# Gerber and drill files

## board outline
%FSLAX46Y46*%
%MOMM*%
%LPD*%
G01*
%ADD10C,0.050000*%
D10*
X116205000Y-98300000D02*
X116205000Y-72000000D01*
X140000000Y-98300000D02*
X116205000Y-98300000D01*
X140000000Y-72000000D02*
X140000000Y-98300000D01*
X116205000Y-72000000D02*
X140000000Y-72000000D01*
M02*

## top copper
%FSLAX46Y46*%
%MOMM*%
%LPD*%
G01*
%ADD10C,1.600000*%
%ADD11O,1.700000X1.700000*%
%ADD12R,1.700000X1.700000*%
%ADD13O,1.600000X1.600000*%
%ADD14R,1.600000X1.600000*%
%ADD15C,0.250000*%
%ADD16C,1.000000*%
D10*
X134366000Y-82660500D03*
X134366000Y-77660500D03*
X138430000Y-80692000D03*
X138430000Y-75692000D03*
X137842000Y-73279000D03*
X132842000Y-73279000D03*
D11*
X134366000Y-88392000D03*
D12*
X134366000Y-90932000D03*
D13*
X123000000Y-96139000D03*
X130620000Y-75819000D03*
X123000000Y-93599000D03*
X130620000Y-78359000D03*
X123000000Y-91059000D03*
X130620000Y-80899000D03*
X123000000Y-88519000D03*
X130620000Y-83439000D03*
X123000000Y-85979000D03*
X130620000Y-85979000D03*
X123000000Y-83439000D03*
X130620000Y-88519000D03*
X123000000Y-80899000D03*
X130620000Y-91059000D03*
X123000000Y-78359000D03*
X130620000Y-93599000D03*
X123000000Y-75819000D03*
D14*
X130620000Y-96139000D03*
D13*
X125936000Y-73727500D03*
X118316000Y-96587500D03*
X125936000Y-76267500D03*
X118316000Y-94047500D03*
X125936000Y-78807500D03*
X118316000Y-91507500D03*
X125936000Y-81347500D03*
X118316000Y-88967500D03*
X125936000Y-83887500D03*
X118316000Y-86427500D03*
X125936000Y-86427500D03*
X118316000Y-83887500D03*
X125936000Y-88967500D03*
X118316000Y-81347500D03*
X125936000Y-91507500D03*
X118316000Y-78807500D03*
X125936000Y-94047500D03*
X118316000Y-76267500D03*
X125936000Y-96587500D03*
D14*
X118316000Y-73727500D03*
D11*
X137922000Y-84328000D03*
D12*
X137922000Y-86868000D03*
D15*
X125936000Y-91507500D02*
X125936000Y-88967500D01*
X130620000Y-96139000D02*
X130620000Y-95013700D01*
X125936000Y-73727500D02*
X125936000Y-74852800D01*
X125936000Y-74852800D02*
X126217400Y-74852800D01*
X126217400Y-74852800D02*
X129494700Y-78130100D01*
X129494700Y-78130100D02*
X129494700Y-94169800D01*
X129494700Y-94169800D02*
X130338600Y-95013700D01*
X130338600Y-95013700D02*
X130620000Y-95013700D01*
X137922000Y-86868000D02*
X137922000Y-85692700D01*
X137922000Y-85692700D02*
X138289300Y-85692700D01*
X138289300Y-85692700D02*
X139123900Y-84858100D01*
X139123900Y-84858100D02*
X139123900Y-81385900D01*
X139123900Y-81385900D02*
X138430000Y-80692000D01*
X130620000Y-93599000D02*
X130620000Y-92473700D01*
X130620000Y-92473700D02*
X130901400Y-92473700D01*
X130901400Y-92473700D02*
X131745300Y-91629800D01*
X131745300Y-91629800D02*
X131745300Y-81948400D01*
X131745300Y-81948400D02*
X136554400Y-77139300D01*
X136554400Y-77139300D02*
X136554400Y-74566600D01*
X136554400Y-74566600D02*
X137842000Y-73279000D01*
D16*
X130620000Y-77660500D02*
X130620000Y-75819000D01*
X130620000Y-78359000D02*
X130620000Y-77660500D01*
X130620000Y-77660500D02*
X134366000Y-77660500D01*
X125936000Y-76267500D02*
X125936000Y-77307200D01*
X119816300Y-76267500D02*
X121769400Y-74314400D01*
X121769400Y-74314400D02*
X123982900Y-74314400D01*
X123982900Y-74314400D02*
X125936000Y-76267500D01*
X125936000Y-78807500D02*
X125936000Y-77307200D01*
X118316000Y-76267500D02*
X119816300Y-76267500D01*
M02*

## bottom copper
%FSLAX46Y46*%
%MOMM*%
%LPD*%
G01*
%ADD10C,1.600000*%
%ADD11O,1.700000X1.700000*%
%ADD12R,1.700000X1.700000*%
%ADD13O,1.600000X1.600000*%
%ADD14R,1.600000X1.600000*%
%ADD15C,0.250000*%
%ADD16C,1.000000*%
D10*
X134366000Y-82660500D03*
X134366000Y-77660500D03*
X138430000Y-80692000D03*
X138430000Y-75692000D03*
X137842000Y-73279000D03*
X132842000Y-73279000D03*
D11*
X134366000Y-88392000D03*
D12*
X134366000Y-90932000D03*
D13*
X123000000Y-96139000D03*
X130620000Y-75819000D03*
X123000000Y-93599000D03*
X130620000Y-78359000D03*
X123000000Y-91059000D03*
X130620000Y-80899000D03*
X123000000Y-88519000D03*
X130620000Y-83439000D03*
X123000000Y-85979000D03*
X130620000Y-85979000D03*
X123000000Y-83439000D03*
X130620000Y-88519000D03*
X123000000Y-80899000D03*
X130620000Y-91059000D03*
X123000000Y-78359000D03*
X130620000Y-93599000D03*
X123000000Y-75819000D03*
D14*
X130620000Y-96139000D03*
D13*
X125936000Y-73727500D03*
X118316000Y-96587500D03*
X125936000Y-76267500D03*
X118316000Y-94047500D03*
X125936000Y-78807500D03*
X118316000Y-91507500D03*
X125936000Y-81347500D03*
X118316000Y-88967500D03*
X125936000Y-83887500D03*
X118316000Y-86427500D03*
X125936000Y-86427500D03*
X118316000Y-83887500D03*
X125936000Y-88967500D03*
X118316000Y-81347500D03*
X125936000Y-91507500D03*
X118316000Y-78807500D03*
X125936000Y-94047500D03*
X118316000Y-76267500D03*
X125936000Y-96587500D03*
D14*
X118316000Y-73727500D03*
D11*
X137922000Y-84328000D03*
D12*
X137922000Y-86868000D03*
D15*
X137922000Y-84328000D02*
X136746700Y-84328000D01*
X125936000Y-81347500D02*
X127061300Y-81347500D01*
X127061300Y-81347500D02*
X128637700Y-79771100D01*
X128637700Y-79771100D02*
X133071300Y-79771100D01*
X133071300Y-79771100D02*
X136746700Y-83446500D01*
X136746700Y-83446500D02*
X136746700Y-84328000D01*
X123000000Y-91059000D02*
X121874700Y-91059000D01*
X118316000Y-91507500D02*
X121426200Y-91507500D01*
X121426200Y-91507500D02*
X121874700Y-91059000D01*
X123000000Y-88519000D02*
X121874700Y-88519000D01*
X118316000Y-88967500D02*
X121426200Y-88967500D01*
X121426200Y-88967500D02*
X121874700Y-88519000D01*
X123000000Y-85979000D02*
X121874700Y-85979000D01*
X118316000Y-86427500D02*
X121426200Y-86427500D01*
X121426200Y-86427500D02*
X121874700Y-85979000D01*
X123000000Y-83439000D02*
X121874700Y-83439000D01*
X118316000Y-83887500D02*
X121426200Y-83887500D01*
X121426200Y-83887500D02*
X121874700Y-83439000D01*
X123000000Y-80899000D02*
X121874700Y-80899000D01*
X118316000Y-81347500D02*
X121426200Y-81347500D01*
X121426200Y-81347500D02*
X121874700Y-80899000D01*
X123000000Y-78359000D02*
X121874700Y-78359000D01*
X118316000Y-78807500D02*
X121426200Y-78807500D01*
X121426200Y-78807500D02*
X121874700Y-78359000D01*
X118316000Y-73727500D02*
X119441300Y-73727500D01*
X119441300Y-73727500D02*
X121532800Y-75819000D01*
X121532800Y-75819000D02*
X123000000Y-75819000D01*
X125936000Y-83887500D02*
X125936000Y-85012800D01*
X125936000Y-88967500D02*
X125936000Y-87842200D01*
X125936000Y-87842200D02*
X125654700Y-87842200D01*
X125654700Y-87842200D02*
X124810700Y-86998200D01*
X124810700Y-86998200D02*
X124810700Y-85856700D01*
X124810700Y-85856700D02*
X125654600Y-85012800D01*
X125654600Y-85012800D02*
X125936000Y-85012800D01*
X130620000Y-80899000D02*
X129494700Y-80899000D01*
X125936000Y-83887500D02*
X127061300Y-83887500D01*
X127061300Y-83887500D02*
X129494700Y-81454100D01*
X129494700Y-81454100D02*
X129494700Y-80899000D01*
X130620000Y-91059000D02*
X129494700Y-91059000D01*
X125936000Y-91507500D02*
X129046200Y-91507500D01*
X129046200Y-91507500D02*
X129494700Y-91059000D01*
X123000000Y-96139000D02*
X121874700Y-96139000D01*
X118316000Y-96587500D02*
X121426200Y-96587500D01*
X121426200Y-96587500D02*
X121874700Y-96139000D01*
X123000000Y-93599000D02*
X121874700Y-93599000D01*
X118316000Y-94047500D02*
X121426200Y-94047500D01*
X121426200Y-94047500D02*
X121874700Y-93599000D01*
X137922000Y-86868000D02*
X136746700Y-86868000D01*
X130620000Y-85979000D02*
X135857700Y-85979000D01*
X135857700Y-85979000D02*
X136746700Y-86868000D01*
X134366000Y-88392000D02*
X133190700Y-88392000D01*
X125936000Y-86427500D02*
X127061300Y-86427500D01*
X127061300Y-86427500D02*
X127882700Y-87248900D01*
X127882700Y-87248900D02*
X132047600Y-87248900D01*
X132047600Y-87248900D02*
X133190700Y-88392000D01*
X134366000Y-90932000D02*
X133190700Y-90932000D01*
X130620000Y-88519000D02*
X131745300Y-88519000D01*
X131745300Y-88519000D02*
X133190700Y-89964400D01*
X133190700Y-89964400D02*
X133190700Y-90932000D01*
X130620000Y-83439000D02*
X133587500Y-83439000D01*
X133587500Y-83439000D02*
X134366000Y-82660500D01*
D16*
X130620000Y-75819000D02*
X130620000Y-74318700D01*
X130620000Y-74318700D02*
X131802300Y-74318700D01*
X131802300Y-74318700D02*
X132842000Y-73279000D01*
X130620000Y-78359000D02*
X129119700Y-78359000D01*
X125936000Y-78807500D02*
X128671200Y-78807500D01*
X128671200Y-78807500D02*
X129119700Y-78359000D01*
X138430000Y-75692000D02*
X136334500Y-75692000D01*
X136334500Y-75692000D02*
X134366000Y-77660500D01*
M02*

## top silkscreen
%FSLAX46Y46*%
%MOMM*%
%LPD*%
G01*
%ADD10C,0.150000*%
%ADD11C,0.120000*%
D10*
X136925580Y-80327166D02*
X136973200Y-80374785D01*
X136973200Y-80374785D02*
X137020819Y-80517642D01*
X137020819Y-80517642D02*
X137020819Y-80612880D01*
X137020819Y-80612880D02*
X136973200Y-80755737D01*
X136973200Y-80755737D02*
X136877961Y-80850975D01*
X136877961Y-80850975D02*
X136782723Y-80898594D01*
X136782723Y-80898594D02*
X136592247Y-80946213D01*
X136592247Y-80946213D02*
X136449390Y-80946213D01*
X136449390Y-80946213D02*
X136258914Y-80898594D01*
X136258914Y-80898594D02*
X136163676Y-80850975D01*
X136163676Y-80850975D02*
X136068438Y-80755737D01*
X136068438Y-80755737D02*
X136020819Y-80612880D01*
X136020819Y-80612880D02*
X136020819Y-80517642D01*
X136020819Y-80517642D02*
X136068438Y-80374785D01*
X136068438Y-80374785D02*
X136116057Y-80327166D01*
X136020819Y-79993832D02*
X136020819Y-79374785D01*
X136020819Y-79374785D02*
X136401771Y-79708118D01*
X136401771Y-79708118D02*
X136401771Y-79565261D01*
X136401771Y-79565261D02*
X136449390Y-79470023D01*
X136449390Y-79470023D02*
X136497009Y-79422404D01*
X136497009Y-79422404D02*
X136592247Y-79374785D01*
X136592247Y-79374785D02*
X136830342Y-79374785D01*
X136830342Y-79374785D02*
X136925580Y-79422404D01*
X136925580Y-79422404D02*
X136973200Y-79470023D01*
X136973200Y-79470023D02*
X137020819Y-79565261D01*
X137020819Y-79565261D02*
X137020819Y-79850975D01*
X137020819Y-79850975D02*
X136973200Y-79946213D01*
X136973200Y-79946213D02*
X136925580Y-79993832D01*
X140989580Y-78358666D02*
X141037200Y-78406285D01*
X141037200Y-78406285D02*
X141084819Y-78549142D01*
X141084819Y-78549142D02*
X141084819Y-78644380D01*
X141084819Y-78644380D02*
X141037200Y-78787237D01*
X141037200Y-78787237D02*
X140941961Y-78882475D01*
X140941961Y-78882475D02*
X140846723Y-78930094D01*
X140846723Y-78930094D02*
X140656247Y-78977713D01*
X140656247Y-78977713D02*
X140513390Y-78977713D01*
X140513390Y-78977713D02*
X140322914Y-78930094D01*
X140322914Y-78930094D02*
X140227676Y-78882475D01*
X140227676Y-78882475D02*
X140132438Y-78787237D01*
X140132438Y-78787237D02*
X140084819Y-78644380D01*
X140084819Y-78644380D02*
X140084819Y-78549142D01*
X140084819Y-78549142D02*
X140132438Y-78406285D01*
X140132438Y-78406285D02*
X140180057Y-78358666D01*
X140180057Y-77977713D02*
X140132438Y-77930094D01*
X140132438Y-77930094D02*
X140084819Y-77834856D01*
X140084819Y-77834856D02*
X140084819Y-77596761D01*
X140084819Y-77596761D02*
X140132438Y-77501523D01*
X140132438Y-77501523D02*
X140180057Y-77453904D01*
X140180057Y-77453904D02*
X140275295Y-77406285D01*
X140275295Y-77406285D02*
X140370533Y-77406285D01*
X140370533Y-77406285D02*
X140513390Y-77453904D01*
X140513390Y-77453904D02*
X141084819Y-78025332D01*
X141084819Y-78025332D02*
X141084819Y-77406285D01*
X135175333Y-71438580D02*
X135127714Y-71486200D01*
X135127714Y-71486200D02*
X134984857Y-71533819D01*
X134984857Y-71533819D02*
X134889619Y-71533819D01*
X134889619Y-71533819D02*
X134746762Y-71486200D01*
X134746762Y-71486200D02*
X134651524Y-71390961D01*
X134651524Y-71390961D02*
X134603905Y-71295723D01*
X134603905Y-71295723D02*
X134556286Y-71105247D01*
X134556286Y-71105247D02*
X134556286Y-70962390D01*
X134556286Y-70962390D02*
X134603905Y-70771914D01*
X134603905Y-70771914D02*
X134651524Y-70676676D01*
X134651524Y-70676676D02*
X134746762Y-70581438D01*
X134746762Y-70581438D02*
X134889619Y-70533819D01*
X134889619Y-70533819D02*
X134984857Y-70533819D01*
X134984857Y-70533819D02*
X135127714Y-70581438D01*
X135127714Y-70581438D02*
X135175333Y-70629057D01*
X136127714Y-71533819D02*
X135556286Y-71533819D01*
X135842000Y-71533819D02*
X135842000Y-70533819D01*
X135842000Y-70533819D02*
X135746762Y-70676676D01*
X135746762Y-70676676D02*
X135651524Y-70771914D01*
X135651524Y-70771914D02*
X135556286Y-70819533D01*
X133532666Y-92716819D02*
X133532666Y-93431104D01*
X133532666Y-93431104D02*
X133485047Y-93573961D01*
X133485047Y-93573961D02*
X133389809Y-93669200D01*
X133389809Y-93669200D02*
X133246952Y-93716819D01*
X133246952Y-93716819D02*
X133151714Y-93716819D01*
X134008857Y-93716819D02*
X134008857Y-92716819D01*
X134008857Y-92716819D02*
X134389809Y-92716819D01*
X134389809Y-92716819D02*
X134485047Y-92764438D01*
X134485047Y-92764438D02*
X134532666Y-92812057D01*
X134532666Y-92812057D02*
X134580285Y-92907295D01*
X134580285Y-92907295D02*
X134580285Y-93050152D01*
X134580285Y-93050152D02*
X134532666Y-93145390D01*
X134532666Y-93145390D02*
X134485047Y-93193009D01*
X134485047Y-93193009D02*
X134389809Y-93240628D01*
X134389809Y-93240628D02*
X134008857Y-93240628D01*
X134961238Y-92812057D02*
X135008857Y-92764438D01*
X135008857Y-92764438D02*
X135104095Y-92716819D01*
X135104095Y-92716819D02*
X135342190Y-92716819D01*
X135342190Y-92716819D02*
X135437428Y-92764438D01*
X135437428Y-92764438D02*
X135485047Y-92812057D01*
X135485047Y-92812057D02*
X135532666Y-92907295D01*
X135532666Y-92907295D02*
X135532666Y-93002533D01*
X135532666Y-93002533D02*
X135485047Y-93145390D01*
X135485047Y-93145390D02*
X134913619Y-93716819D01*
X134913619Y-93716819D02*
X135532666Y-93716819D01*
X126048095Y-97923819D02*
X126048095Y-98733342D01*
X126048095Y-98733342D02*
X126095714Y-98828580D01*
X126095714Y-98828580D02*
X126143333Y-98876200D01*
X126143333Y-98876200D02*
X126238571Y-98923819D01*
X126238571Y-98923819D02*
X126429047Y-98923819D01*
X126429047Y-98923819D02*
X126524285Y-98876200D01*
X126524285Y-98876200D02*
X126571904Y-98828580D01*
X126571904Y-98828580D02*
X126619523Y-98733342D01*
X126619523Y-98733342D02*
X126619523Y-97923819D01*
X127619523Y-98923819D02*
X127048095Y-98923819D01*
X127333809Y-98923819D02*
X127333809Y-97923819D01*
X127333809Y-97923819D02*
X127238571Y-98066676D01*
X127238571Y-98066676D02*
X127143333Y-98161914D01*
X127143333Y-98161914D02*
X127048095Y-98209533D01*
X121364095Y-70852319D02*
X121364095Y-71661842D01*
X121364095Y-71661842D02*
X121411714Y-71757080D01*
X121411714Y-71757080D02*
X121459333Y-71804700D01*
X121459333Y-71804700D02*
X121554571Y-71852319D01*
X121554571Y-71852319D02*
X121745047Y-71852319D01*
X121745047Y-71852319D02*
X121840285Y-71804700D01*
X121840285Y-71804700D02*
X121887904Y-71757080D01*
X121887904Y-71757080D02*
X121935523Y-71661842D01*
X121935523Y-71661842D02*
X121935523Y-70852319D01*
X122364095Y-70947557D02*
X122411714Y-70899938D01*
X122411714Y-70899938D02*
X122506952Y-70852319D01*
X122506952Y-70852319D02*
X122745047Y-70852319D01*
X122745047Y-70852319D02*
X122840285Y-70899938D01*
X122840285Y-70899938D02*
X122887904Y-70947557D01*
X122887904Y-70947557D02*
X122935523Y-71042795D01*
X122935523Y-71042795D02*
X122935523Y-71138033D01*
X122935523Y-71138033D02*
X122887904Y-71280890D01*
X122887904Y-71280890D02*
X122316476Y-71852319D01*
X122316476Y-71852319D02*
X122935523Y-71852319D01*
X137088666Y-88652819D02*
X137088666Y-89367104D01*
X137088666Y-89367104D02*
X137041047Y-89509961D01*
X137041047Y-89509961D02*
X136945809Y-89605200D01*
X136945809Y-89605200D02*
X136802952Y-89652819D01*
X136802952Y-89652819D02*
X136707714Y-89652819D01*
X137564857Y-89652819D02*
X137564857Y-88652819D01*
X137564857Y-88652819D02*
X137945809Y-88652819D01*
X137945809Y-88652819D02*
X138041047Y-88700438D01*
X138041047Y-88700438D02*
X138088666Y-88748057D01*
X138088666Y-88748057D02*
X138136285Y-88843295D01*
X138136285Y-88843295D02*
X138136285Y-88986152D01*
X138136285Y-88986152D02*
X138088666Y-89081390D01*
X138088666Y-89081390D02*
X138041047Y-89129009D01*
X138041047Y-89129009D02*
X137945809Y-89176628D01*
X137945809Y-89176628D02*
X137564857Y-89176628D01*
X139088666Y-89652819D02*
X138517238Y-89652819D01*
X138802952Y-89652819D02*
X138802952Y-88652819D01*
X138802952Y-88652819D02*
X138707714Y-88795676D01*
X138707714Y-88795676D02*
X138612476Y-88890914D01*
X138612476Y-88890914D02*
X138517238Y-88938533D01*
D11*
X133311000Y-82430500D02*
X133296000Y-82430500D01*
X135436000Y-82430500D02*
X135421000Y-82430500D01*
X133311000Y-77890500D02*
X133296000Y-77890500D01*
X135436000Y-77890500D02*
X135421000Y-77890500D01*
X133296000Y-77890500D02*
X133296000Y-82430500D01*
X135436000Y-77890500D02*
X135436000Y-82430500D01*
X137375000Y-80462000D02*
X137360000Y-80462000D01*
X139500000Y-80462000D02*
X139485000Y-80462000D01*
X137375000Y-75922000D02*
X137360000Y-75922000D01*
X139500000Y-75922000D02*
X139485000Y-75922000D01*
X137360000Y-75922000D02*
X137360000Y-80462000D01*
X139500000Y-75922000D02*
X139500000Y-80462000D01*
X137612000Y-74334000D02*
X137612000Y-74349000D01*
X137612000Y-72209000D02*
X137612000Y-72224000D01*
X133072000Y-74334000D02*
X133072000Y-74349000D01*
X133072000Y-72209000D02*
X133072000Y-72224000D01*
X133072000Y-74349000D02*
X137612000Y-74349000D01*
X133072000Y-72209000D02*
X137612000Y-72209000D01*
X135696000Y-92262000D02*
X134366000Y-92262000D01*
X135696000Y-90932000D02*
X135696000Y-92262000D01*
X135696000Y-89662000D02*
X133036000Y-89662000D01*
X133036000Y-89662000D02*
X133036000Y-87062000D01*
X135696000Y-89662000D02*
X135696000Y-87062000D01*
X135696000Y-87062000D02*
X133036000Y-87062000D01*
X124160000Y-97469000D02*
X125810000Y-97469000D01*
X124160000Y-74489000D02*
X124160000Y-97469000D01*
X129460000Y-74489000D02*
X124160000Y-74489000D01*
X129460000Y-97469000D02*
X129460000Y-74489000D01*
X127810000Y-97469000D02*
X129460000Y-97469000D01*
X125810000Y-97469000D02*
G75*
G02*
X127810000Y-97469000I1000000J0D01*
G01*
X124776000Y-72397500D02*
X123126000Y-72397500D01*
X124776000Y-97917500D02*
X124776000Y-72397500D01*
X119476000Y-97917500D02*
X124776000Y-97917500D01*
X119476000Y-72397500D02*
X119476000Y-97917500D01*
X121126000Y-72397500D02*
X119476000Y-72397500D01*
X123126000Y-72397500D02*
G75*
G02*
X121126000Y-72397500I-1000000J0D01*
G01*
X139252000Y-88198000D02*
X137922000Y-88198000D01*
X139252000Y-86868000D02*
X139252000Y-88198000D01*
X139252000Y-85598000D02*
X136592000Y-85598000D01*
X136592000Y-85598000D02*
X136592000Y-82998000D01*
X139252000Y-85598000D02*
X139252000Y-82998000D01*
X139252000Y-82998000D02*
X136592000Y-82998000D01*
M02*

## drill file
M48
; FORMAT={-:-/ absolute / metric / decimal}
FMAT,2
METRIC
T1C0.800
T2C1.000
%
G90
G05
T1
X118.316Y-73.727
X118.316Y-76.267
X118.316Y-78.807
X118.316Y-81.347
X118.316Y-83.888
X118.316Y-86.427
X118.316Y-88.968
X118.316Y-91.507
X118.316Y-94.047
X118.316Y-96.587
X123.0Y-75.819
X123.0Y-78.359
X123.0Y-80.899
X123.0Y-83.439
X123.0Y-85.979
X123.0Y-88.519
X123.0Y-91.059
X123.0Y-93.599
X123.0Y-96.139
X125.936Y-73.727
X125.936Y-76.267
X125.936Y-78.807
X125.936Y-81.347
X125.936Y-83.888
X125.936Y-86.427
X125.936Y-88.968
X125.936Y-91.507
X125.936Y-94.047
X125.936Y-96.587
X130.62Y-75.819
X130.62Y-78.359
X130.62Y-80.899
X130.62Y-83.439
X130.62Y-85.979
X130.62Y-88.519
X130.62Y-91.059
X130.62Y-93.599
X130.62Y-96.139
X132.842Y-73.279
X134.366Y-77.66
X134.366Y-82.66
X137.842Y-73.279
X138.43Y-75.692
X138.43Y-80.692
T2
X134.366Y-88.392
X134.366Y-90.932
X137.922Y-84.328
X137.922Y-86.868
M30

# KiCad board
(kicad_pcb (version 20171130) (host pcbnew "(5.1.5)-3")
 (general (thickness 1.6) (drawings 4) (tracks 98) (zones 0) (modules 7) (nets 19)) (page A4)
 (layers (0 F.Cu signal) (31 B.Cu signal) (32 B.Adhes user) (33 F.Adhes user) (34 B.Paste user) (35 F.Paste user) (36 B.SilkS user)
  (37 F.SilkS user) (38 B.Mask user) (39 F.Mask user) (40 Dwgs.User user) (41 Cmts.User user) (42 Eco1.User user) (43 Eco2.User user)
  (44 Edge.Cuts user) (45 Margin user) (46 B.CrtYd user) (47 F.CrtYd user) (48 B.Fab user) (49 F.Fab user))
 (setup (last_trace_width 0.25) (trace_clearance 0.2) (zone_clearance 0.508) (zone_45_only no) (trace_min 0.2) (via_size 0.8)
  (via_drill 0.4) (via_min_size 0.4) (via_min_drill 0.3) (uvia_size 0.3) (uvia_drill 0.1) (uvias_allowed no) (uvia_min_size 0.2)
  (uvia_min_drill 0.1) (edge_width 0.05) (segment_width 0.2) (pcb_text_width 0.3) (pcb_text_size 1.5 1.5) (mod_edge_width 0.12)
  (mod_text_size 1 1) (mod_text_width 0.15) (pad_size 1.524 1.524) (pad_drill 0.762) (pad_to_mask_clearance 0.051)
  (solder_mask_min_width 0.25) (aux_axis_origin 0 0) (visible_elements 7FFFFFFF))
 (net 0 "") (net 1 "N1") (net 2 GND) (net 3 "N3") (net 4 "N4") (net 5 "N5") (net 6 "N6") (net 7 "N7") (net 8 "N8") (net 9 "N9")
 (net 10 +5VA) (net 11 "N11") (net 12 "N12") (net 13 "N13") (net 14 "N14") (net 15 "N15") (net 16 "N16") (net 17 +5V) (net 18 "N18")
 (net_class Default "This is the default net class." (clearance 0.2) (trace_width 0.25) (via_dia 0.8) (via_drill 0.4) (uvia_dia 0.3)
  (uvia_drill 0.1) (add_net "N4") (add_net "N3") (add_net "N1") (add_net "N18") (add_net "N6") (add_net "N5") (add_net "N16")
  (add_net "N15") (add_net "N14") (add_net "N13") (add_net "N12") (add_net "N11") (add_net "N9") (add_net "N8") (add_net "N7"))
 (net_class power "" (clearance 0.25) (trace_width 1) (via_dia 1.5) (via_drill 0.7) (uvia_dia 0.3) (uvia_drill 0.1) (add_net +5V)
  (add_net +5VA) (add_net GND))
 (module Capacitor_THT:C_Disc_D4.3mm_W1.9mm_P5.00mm (layer F.Cu) (at 134.366 77.6605 270)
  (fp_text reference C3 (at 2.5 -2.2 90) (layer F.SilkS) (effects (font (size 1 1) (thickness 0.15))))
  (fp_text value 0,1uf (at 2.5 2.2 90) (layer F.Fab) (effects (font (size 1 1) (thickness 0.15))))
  (fp_line (start 4.77 1.055) (end 4.77 1.07) (layer F.SilkS) (width 0.12))
  (fp_line (start 4.77 -1.07) (end 4.77 -1.055) (layer F.SilkS) (width 0.12))
  (fp_line (start 0.23 1.055) (end 0.23 1.07) (layer F.SilkS) (width 0.12))
  (fp_line (start 0.23 -1.07) (end 0.23 -1.055) (layer F.SilkS) (width 0.12))
  (fp_line (start 0.23 1.07) (end 4.77 1.07) (layer F.SilkS) (width 0.12))
  (fp_line (start 0.23 -1.07) (end 4.77 -1.07) (layer F.SilkS) (width 0.12))
  (pad 2 thru_hole circle (at 5 0 270) (size 1.6 1.6) (drill 0.8) (layers *.Cu *.Mask) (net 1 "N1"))
  (pad 1 thru_hole circle (at 0 0 270) (size 1.6 1.6) (drill 0.8) (layers *.Cu *.Mask) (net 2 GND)))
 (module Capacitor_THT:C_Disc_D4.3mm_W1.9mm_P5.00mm (layer F.Cu) (at 138.43 75.692 270)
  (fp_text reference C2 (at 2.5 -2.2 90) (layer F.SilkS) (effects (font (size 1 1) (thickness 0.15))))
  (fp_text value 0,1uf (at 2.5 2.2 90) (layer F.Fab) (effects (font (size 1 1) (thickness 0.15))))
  (fp_line (start 4.77 1.055) (end 4.77 1.07) (layer F.SilkS) (width 0.12))
  (fp_line (start 4.77 -1.07) (end 4.77 -1.055) (layer F.SilkS) (width 0.12))
  (fp_line (start 0.23 1.055) (end 0.23 1.07) (layer F.SilkS) (width 0.12))
  (fp_line (start 0.23 -1.07) (end 0.23 -1.055) (layer F.SilkS) (width 0.12))
  (fp_line (start 0.23 1.07) (end 4.77 1.07) (layer F.SilkS) (width 0.12))
  (fp_line (start 0.23 -1.07) (end 4.77 -1.07) (layer F.SilkS) (width 0.12))
  (pad 2 thru_hole circle (at 5 0 270) (size 1.6 1.6) (drill 0.8) (layers *.Cu *.Mask) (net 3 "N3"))
  (pad 1 thru_hole circle (at 0 0 270) (size 1.6 1.6) (drill 0.8) (layers *.Cu *.Mask) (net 2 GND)))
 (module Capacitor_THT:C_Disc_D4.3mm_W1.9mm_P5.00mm (layer F.Cu) (at 132.842 73.279)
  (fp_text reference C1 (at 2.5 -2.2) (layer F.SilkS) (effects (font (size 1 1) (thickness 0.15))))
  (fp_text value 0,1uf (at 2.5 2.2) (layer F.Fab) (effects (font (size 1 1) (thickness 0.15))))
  (fp_line (start 4.77 1.055) (end 4.77 1.07) (layer F.SilkS) (width 0.12))
  (fp_line (start 4.77 -1.07) (end 4.77 -1.055) (layer F.SilkS) (width 0.12))
  (fp_line (start 0.23 1.055) (end 0.23 1.07) (layer F.SilkS) (width 0.12))
  (fp_line (start 0.23 -1.07) (end 0.23 -1.055) (layer F.SilkS) (width 0.12))
  (fp_line (start 0.23 1.07) (end 4.77 1.07) (layer F.SilkS) (width 0.12))
  (fp_line (start 0.23 -1.07) (end 4.77 -1.07) (layer F.SilkS) (width 0.12))
  (pad 2 thru_hole circle (at 5 0) (size 1.6 1.6) (drill 0.8) (layers *.Cu *.Mask) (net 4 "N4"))
  (pad 1 thru_hole circle (at 0 0) (size 1.6 1.6) (drill 0.8) (layers *.Cu *.Mask) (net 2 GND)))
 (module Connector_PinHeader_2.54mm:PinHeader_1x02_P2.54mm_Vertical (layer F.Cu) (at 134.366 90.932 180)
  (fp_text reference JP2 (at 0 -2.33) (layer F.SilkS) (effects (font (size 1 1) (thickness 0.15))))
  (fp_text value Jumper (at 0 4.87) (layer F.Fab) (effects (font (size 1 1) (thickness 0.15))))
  (fp_line (start -1.33 -1.33) (end 0 -1.33) (layer F.SilkS) (width 0.12))
  (fp_line (start -1.33 0) (end -1.33 -1.33) (layer F.SilkS) (width 0.12))
  (fp_line (start -1.33 1.27) (end 1.33 1.27) (layer F.SilkS) (width 0.12))
  (fp_line (start 1.33 1.27) (end 1.33 3.87) (layer F.SilkS) (width 0.12))
  (fp_line (start -1.33 1.27) (end -1.33 3.87) (layer F.SilkS) (width 0.12))
  (fp_line (start -1.33 3.87) (end 1.33 3.87) (layer F.SilkS) (width 0.12))
  (pad 2 thru_hole oval (at 0 2.54 180) (size 1.7 1.7) (drill 1) (layers *.Cu *.Mask) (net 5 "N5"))
  (pad 1 thru_hole rect (at 0 0 180) (size 1.7 1.7) (drill 1) (layers *.Cu *.Mask) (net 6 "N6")))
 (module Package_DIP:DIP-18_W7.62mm (layer F.Cu) (at 130.62 96.139 180)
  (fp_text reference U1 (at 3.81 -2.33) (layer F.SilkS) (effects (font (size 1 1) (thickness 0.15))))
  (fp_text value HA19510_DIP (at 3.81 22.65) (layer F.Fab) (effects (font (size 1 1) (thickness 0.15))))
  (fp_line (start 6.46 -1.33) (end 4.81 -1.33) (layer F.SilkS) (width 0.12))
  (fp_line (start 6.46 21.65) (end 6.46 -1.33) (layer F.SilkS) (width 0.12))
  (fp_line (start 1.16 21.65) (end 6.46 21.65) (layer F.SilkS) (width 0.12))
  (fp_line (start 1.16 -1.33) (end 1.16 21.65) (layer F.SilkS) (width 0.12))
  (fp_line (start 2.81 -1.33) (end 1.16 -1.33) (layer F.SilkS) (width 0.12))
  (fp_arc (start 3.81 -1.33) (end 2.81 -1.33) (angle -180) (layer F.SilkS) (width 0.12))
  (pad 18 thru_hole oval (at 7.62 0 180) (size 1.6 1.6) (drill 0.8) (layers *.Cu *.Mask) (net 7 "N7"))
  (pad 9 thru_hole oval (at 0 20.32 180) (size 1.6 1.6) (drill 0.8) (layers *.Cu *.Mask) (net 2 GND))
  (pad 17 thru_hole oval (at 7.62 2.54 180) (size 1.6 1.6) (drill 0.8) (layers *.Cu *.Mask) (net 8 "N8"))
  (pad 8 thru_hole oval (at 0 17.78 180) (size 1.6 1.6) (drill 0.8) (layers *.Cu *.Mask) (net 2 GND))
  (pad 16 thru_hole oval (at 7.62 5.08 180) (size 1.6 1.6) (drill 0.8) (layers *.Cu *.Mask) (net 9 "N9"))
  (pad 7 thru_hole oval (at 0 15.24 180) (size 1.6 1.6) (drill 0.8) (layers *.Cu *.Mask) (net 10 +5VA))
  (pad 15 thru_hole oval (at 7.62 7.62 180) (size 1.6 1.6) (drill 0.8) (layers *.Cu *.Mask) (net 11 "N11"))
  (pad 6 thru_hole oval (at 0 12.7 180) (size 1.6 1.6) (drill 0.8) (layers *.Cu *.Mask) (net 1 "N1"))
  (pad 14 thru_hole oval (at 7.62 10.16 180) (size 1.6 1.6) (drill 0.8) (layers *.Cu *.Mask) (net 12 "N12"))
  (pad 5 thru_hole oval (at 0 10.16 180) (size 1.6 1.6) (drill 0.8) (layers *.Cu *.Mask) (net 3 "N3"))
  (pad 13 thru_hole oval (at 7.62 12.7 180) (size 1.6 1.6) (drill 0.8) (layers *.Cu *.Mask) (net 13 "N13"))
  (pad 4 thru_hole oval (at 0 7.62 180) (size 1.6 1.6) (drill 0.8) (layers *.Cu *.Mask) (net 6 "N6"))
  (pad 12 thru_hole oval (at 7.62 15.24 180) (size 1.6 1.6) (drill 0.8) (layers *.Cu *.Mask) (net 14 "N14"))
  (pad 3 thru_hole oval (at 0 5.08 180) (size 1.6 1.6) (drill 0.8) (layers *.Cu *.Mask) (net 10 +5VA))
  (pad 11 thru_hole oval (at 7.62 17.78 180) (size 1.6 1.6) (drill 0.8) (layers *.Cu *.Mask) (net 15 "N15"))
  (pad 2 thru_hole oval (at 0 2.54 180) (size 1.6 1.6) (drill 0.8) (layers *.Cu *.Mask) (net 4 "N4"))
  (pad 10 thru_hole oval (at 7.62 20.32 180) (size 1.6 1.6) (drill 0.8) (layers *.Cu *.Mask) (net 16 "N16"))
  (pad 1 thru_hole rect (at 0 0 180) (size 1.6 1.6) (drill 0.8) (layers *.Cu *.Mask) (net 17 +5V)))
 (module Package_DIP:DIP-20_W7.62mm (layer F.Cu) (at 118.316 73.7275)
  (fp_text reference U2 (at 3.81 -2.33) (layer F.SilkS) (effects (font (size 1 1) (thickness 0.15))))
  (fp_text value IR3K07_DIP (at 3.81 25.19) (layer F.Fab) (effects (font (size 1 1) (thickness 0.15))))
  (fp_line (start 6.46 -1.33) (end 4.81 -1.33) (layer F.SilkS) (width 0.12))
  (fp_line (start 6.46 24.19) (end 6.46 -1.33) (layer F.SilkS) (width 0.12))
  (fp_line (start 1.16 24.19) (end 6.46 24.19) (layer F.SilkS) (width 0.12))
  (fp_line (start 1.16 -1.33) (end 1.16 24.19) (layer F.SilkS) (width 0.12))
  (fp_line (start 2.81 -1.33) (end 1.16 -1.33) (layer F.SilkS) (width 0.12))
  (fp_arc (start 3.81 -1.33) (end 2.81 -1.33) (angle -180) (layer F.SilkS) (width 0.12))
  (pad 20 thru_hole oval (at 7.62 0) (size 1.6 1.6) (drill 0.8) (layers *.Cu *.Mask) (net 17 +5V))
  (pad 10 thru_hole oval (at 0 22.86) (size 1.6 1.6) (drill 0.8) (layers *.Cu *.Mask) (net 7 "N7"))
  (pad 19 thru_hole oval (at 7.62 2.54) (size 1.6 1.6) (drill 0.8) (layers *.Cu *.Mask) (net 2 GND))
  (pad 9 thru_hole oval (at 0 20.32) (size 1.6 1.6) (drill 0.8) (layers *.Cu *.Mask) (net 8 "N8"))
  (pad 18 thru_hole oval (at 7.62 5.08) (size 1.6 1.6) (drill 0.8) (layers *.Cu *.Mask) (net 2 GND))
  (pad 8 thru_hole oval (at 0 17.78) (size 1.6 1.6) (drill 0.8) (layers *.Cu *.Mask) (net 9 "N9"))
  (pad 17 thru_hole oval (at 7.62 7.62) (size 1.6 1.6) (drill 0.8) (layers *.Cu *.Mask) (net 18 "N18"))
  (pad 7 thru_hole oval (at 0 15.24) (size 1.6 1.6) (drill 0.8) (layers *.Cu *.Mask) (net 11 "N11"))
  (pad 16 thru_hole oval (at 7.62 10.16) (size 1.6 1.6) (drill 0.8) (layers *.Cu *.Mask) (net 10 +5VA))
  (pad 6 thru_hole oval (at 0 12.7) (size 1.6 1.6) (drill 0.8) (layers *.Cu *.Mask) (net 12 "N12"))
  (pad 15 thru_hole oval (at 7.62 12.7) (size 1.6 1.6) (drill 0.8) (layers *.Cu *.Mask) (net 5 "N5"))
  (pad 5 thru_hole oval (at 0 10.16) (size 1.6 1.6) (drill 0.8) (layers *.Cu *.Mask) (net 13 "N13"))
  (pad 14 thru_hole oval (at 7.62 15.24) (size 1.6 1.6) (drill 0.8) (layers *.Cu *.Mask) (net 10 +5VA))
  (pad 4 thru_hole oval (at 0 7.62) (size 1.6 1.6) (drill 0.8) (layers *.Cu *.Mask) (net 14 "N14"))
  (pad 13 thru_hole oval (at 7.62 17.78) (size 1.6 1.6) (drill 0.8) (layers *.Cu *.Mask) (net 10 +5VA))
  (pad 3 thru_hole oval (at 0 5.08) (size 1.6 1.6) (drill 0.8) (layers *.Cu *.Mask) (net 15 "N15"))
  (pad 12 thru_hole oval (at 7.62 20.32) (size 1.6 1.6) (drill 0.8) (layers *.Cu *.Mask))
  (pad 2 thru_hole oval (at 0 2.54) (size 1.6 1.6) (drill 0.8) (layers *.Cu *.Mask) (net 2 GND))
  (pad 11 thru_hole oval (at 7.62 22.86) (size 1.6 1.6) (drill 0.8) (layers *.Cu *.Mask))
  (pad 1 thru_hole rect (at 0 0) (size 1.6 1.6) (drill 0.8) (layers *.Cu *.Mask) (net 16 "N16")))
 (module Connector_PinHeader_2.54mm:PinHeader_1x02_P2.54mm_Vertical (layer F.Cu) (at 137.922 86.868 180)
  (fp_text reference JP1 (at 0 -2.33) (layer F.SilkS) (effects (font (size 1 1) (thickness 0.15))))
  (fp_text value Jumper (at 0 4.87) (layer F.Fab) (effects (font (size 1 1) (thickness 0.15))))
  (fp_line (start -1.33 -1.33) (end 0 -1.33) (layer F.SilkS) (width 0.12))
  (fp_line (start -1.33 0) (end -1.33 -1.33) (layer F.SilkS) (width 0.12))
  (fp_line (start -1.33 1.27) (end 1.33 1.27) (layer F.SilkS) (width 0.12))
  (fp_line (start 1.33 1.27) (end 1.33 3.87) (layer F.SilkS) (width 0.12))
  (fp_line (start -1.33 1.27) (end -1.33 3.87) (layer F.SilkS) (width 0.12))
  (fp_line (start -1.33 3.87) (end 1.33 3.87) (layer F.SilkS) (width 0.12))
  (pad 2 thru_hole oval (at 0 2.54 180) (size 1.7 1.7) (drill 1) (layers *.Cu *.Mask) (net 18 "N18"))
  (pad 1 thru_hole rect (at 0 0 180) (size 1.7 1.7) (drill 1) (layers *.Cu *.Mask) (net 3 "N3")))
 (gr_line (start 116.205 98.3) (end 116.205 72) (layer Edge.Cuts) (width 0.05))
 (gr_line (start 140 98.3) (end 116.205 98.3) (layer Edge.Cuts) (width 0.05))
 (gr_line (start 140 72) (end 140 98.3) (layer Edge.Cuts) (width 0.05))
 (gr_line (start 116.205 72) (end 140 72) (layer Edge.Cuts) (width 0.05))
 (segment (start 137.922 84.328) (end 136.7467 84.328) (width 0.25) (layer B.Cu) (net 18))
 (segment (start 125.936 81.3475) (end 127.0613 81.3475) (width 0.25) (layer B.Cu) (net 18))
 (segment (start 127.0613 81.3475) (end 128.6377 79.7711) (width 0.25) (layer B.Cu) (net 18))
 (segment (start 128.6377 79.7711) (end 133.0713 79.7711) (width 0.25) (layer B.Cu) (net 18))
 (segment (start 133.0713 79.7711) (end 136.7467 83.4465) (width 0.25) (layer B.Cu) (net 18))
 (segment (start 136.7467 83.4465) (end 136.7467 84.328) (width 0.25) (layer B.Cu) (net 18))
 (segment (start 123 91.059) (end 121.8747 91.059) (width 0.25) (layer B.Cu) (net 9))
 (segment (start 118.316 91.5075) (end 121.4262 91.5075) (width 0.25) (layer B.Cu) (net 9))
 (segment (start 121.4262 91.5075) (end 121.8747 91.059) (width 0.25) (layer B.Cu) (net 9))
 (segment (start 123 88.519) (end 121.8747 88.519) (width 0.25) (layer B.Cu) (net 11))
 (segment (start 118.316 88.9675) (end 121.4262 88.9675) (width 0.25) (layer B.Cu) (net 11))
 (segment (start 121.4262 88.9675) (end 121.8747 88.519) (width 0.25) (layer B.Cu) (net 11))
 (segment (start 123 85.979) (end 121.8747 85.979) (width 0.25) (layer B.Cu) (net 12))
 (segment (start 118.316 86.4275) (end 121.4262 86.4275) (width 0.25) (layer B.Cu) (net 12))
 (segment (start 121.4262 86.4275) (end 121.8747 85.979) (width 0.25) (layer B.Cu) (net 12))
 (segment (start 123 83.439) (end 121.8747 83.439) (width 0.25) (layer B.Cu) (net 13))
 (segment (start 118.316 83.8875) (end 121.4262 83.8875) (width 0.25) (layer B.Cu) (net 13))
 (segment (start 121.4262 83.8875) (end 121.8747 83.439) (width 0.25) (layer B.Cu) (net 13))
 (segment (start 123 80.899) (end 121.8747 80.899) (width 0.25) (layer B.Cu) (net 14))
 (segment (start 118.316 81.3475) (end 121.4262 81.3475) (width 0.25) (layer B.Cu) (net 14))
 (segment (start 121.4262 81.3475) (end 121.8747 80.899) (width 0.25) (layer B.Cu) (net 14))
 (segment (start 123 78.359) (end 121.8747 78.359) (width 0.25) (layer B.Cu) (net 15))
 (segment (start 118.316 78.8075) (end 121.4262 78.8075) (width 0.25) (layer B.Cu) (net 15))
 (segment (start 121.4262 78.8075) (end 121.8747 78.359) (width 0.25) (layer B.Cu) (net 15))
 (segment (start 118.316 73.7275) (end 119.4413 73.7275) (width 0.25) (layer B.Cu) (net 16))
 (segment (start 119.4413 73.7275) (end 121.5328 75.819) (width 0.25) (layer B.Cu) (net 16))
 (segment (start 121.5328 75.819) (end 123 75.819) (width 0.25) (layer B.Cu) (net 16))
 (segment (start 125.936 83.8875) (end 125.936 85.0128) (width 0.25) (layer B.Cu) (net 10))
 (segment (start 125.936 88.9675) (end 125.936 87.8422) (width 0.25) (layer B.Cu) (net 10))
 (segment (start 125.936 87.8422) (end 125.6547 87.8422) (width 0.25) (layer B.Cu) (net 10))
 (segment (start 125.6547 87.8422) (end 124.8107 86.9982) (width 0.25) (layer B.Cu) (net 10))
 (segment (start 124.8107 86.9982) (end 124.8107 85.8567) (width 0.25) (layer B.Cu) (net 10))
 (segment (start 124.8107 85.8567) (end 125.6546 85.0128) (width 0.25) (layer B.Cu) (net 10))
 (segment (start 125.6546 85.0128) (end 125.936 85.0128) (width 0.25) (layer B.Cu) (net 10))
 (segment (start 130.62 80.899) (end 129.4947 80.899) (width 0.25) (layer B.Cu) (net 10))
 (segment (start 125.936 83.8875) (end 127.0613 83.8875) (width 0.25) (layer B.Cu) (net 10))
 (segment (start 127.0613 83.8875) (end 129.4947 81.4541) (width 0.25) (layer B.Cu) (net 10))
 (segment (start 129.4947 81.4541) (end 129.4947 80.899) (width 0.25) (layer B.Cu) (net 10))
 (segment (start 130.62 91.059) (end 129.4947 91.059) (width 0.25) (layer B.Cu) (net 10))
 (segment (start 125.936 91.5075) (end 129.0462 91.5075) (width 0.25) (layer B.Cu) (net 10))
 (segment (start 129.0462 91.5075) (end 129.4947 91.059) (width 0.25) (layer B.Cu) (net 10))
 (segment (start 125.936 91.5075) (end 125.936 88.9675) (width 0.25) (layer F.Cu) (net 10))
 (segment (start 130.62 96.139) (end 130.62 95.0137) (width 0.25) (layer F.Cu) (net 17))
 (segment (start 125.936 73.7275) (end 125.936 74.8528) (width 0.25) (layer F.Cu) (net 17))
 (segment (start 125.936 74.8528) (end 126.2174 74.8528) (width 0.25) (layer F.Cu) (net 17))
 (segment (start 126.2174 74.8528) (end 129.4947 78.1301) (width 0.25) (layer F.Cu) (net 17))
 (segment (start 129.4947 78.1301) (end 129.4947 94.1698) (width 0.25) (layer F.Cu) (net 17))
 (segment (start 129.4947 94.1698) (end 130.3386 95.0137) (width 0.25) (layer F.Cu) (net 17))
 (segment (start 130.3386 95.0137) (end 130.62 95.0137) (width 0.25) (layer F.Cu) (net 17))
 (segment (start 123 96.139) (end 121.8747 96.139) (width 0.25) (layer B.Cu) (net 7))
 (segment (start 118.316 96.5875) (end 121.4262 96.5875) (width 0.25) (layer B.Cu) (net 7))
 (segment (start 121.4262 96.5875) (end 121.8747 96.139) (width 0.25) (layer B.Cu) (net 7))
 (segment (start 123 93.599) (end 121.8747 93.599) (width 0.25) (layer B.Cu) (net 8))
 (segment (start 118.316 94.0475) (end 121.4262 94.0475) (width 0.25) (layer B.Cu) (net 8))
 (segment (start 121.4262 94.0475) (end 121.8747 93.599) (width 0.25) (layer B.Cu) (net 8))
 (segment (start 137.922 86.868) (end 137.922 85.6927) (width 0.25) (layer F.Cu) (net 3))
 (segment (start 137.922 85.6927) (end 138.2893 85.6927) (width 0.25) (layer F.Cu) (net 3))
 (segment (start 138.2893 85.6927) (end 139.1239 84.8581) (width 0.25) (layer F.Cu) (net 3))
 (segment (start 139.1239 84.8581) (end 139.1239 81.3859) (width 0.25) (layer F.Cu) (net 3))
 (segment (start 139.1239 81.3859) (end 138.43 80.692) (width 0.25) (layer F.Cu) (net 3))
 (segment (start 137.922 86.868) (end 136.7467 86.868) (width 0.25) (layer B.Cu) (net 3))
 (segment (start 130.62 85.979) (end 135.8577 85.979) (width 0.25) (layer B.Cu) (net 3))
 (segment (start 135.8577 85.979) (end 136.7467 86.868) (width 0.25) (layer B.Cu) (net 3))
 (segment (start 134.366 88.392) (end 133.1907 88.392) (width 0.25) (layer B.Cu) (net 5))
 (segment (start 125.936 86.4275) (end 127.0613 86.4275) (width 0.25) (layer B.Cu) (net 5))
 (segment (start 127.0613 86.4275) (end 127.8827 87.2489) (width 0.25) (layer B.Cu) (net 5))
 (segment (start 127.8827 87.2489) (end 132.0476 87.2489) (width 0.25) (layer B.Cu) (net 5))
 (segment (start 132.0476 87.2489) (end 133.1907 88.392) (width 0.25) (layer B.Cu) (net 5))
 (segment (start 134.366 90.932) (end 133.1907 90.932) (width 0.25) (layer B.Cu) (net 6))
 (segment (start 130.62 88.519) (end 131.7453 88.519) (width 0.25) (layer B.Cu) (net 6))
 (segment (start 131.7453 88.519) (end 133.1907 89.9644) (width 0.25) (layer B.Cu) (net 6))
 (segment (start 133.1907 89.9644) (end 133.1907 90.932) (width 0.25) (layer B.Cu) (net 6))
 (segment (start 130.62 93.599) (end 130.62 92.4737) (width 0.25) (layer F.Cu) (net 4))
 (segment (start 130.62 92.4737) (end 130.9014 92.4737) (width 0.25) (layer F.Cu) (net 4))
 (segment (start 130.9014 92.4737) (end 131.7453 91.6298) (width 0.25) (layer F.Cu) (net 4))
 (segment (start 131.7453 91.6298) (end 131.7453 81.9484) (width 0.25) (layer F.Cu) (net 4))
 (segment (start 131.7453 81.9484) (end 136.5544 77.1393) (width 0.25) (layer F.Cu) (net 4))
 (segment (start 136.5544 77.1393) (end 136.5544 74.5666) (width 0.25) (layer F.Cu) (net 4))
 (segment (start 136.5544 74.5666) (end 137.842 73.279) (width 0.25) (layer F.Cu) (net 4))
 (segment (start 130.62 83.439) (end 133.5875 83.439) (width 0.25) (layer B.Cu) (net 1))
 (segment (start 133.5875 83.439) (end 134.366 82.6605) (width 0.25) (layer B.Cu) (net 1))
 (segment (start 130.62 77.6605) (end 130.62 75.819) (width 1) (layer F.Cu) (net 2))
 (segment (start 130.62 78.359) (end 130.62 77.6605) (width 1) (layer F.Cu) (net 2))
 (segment (start 130.62 77.6605) (end 134.366 77.6605) (width 1) (layer F.Cu) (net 2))
 (segment (start 130.62 75.819) (end 130.62 74.3187) (width 1) (layer B.Cu) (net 2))
 (segment (start 130.62 74.3187) (end 131.8023 74.3187) (width 1) (layer B.Cu) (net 2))
 (segment (start 131.8023 74.3187) (end 132.842 73.279) (width 1) (layer B.Cu) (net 2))
 (segment (start 130.62 78.359) (end 129.1197 78.359) (width 1) (layer B.Cu) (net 2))
 (segment (start 125.936 78.8075) (end 128.6712 78.8075) (width 1) (layer B.Cu) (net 2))
 (segment (start 128.6712 78.8075) (end 129.1197 78.359) (width 1) (layer B.Cu) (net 2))
 (segment (start 125.936 76.2675) (end 125.936 77.3072) (width 1) (layer F.Cu) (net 2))
 (segment (start 119.8163 76.2675) (end 121.7694 74.3144) (width 1) (layer F.Cu) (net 2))
 (segment (start 121.7694 74.3144) (end 123.9829 74.3144) (width 1) (layer F.Cu) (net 2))
 (segment (start 123.9829 74.3144) (end 125.936 76.2675) (width 1) (layer F.Cu) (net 2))
 (segment (start 125.936 78.8075) (end 125.936 77.3072) (width 1) (layer F.Cu) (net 2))
 (segment (start 138.43 75.692) (end 136.3345 75.692) (width 1) (layer B.Cu) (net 2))
 (segment (start 136.3345 75.692) (end 134.366 77.6605) (width 1) (layer B.Cu) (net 2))
 (segment (start 118.316 76.2675) (end 119.8163 76.2675) (width 1) (layer F.Cu) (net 2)))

